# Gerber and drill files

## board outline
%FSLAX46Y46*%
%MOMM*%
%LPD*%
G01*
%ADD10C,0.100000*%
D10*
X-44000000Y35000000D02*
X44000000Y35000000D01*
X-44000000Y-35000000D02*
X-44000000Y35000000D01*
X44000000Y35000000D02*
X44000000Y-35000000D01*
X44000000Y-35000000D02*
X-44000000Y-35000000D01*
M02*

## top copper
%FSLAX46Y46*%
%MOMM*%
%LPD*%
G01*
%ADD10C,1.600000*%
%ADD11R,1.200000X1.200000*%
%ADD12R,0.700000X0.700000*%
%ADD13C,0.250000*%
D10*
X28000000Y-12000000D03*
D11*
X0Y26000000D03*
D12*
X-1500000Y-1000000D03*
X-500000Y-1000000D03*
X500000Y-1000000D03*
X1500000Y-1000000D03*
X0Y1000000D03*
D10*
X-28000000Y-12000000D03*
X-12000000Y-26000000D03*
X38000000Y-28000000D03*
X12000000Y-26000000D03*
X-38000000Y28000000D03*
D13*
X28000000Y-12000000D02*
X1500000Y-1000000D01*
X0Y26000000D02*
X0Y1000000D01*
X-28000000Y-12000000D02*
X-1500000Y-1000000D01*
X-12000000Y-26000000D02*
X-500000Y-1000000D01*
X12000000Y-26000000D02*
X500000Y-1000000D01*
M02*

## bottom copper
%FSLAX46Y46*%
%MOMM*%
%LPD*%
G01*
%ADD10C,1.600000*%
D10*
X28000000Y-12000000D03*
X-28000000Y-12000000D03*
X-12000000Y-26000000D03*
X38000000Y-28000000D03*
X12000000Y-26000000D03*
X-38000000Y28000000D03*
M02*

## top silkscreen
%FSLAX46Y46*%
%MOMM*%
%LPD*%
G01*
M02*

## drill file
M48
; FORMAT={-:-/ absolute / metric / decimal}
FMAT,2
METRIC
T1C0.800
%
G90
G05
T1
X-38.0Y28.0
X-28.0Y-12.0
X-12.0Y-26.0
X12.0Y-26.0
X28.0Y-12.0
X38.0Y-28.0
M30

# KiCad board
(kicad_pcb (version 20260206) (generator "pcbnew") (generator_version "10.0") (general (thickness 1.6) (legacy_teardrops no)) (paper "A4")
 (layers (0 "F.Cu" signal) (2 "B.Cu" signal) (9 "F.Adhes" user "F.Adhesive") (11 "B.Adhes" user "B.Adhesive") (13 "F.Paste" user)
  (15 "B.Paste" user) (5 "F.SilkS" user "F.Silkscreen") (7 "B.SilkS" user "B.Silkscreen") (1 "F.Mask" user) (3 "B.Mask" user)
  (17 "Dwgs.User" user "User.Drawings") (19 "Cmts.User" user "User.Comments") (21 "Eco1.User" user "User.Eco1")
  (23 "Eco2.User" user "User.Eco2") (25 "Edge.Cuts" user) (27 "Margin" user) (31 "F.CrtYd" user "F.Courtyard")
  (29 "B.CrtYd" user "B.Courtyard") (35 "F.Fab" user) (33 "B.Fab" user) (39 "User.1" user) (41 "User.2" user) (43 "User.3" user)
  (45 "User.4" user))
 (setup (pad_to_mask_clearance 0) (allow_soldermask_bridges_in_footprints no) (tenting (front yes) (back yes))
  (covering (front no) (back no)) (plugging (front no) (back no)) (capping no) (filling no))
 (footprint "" (layer "F.Cu") (at 28 12)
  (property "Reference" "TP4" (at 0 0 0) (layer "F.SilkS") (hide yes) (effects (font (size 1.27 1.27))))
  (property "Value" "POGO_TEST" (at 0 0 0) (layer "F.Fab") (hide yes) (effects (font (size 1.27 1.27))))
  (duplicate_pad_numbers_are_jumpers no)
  (pad "1" thru_hole circle (at 0 0) (size 1.6 1.6) (drill 0.8) (layers "*.Cu" "*.Mask") (remove_unused_layers no) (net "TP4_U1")))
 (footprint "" (layer "F.Cu") (at 0 -26)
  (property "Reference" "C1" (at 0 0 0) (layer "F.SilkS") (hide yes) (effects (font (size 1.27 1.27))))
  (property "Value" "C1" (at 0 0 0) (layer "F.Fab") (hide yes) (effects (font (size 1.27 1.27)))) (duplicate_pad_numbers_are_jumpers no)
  (pad "1" smd rect (at 0 0) (size 1.2 1.2) (layers "F.Cu" "F.Mask" "F.Paste") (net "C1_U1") (thermal_bridge_angle 45)))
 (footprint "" (layer "F.Cu") (at 0 0)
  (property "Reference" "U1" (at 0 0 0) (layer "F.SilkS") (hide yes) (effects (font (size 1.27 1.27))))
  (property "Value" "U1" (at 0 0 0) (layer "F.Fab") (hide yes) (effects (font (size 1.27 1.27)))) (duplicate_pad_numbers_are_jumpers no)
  (pad "1" smd rect (at -1.5 1) (size 0.7 0.7) (layers "F.Cu" "F.Mask" "F.Paste") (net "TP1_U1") (thermal_bridge_angle 45))
  (pad "2" smd rect (at -0.5 1) (size 0.7 0.7) (layers "F.Cu" "F.Mask" "F.Paste") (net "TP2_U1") (thermal_bridge_angle 45))
  (pad "3" smd rect (at 0.5 1) (size 0.7 0.7) (layers "F.Cu" "F.Mask" "F.Paste") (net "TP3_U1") (thermal_bridge_angle 45))
  (pad "4" smd rect (at 1.5 1) (size 0.7 0.7) (layers "F.Cu" "F.Mask" "F.Paste") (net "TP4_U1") (thermal_bridge_angle 45))
  (pad "5" smd rect (at 0 -1) (size 0.7 0.7) (layers "F.Cu" "F.Mask" "F.Paste") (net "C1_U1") (thermal_bridge_angle 45)))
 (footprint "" (layer "F.Cu") (at -28 12)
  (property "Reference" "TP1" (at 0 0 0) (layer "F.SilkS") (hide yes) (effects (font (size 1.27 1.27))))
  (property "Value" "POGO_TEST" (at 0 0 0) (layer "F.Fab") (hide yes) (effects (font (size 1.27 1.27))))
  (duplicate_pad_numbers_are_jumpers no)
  (pad "1" thru_hole circle (at 0 0) (size 1.6 1.6) (drill 0.8) (layers "*.Cu" "*.Mask") (remove_unused_layers no) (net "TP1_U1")))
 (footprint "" (layer "F.Cu") (at -12 26)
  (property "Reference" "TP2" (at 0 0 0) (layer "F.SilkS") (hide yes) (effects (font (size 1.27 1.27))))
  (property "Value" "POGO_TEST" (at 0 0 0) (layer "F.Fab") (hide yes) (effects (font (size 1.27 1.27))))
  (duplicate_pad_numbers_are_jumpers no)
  (pad "1" thru_hole circle (at 0 0) (size 1.6 1.6) (drill 0.8) (layers "*.Cu" "*.Mask") (remove_unused_layers no) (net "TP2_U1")))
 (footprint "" (layer "F.Cu") (at 38 28)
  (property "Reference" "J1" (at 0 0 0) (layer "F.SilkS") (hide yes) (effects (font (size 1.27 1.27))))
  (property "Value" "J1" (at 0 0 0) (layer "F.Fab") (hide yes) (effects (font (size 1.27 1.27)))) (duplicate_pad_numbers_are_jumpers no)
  (pad "1" thru_hole circle (at 0 0) (size 1.6 1.6) (drill 0.8) (layers "*.Cu" "*.Mask") (remove_unused_layers no) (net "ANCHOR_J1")))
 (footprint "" (layer "F.Cu") (at 12 26)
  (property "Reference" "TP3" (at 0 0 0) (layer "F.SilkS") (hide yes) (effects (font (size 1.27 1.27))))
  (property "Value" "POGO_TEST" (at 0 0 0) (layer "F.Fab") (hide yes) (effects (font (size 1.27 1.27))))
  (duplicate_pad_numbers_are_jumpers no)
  (pad "1" thru_hole circle (at 0 0) (size 1.6 1.6) (drill 0.8) (layers "*.Cu" "*.Mask") (remove_unused_layers no) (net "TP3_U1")))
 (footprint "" (layer "F.Cu") (at -38 -28)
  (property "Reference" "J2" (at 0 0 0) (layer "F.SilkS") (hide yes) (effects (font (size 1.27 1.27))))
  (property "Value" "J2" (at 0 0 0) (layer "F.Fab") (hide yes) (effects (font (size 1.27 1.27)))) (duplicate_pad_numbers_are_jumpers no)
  (pad "1" thru_hole circle (at 0 0) (size 1.6 1.6) (drill 0.8) (layers "*.Cu" "*.Mask") (remove_unused_layers no) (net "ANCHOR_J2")))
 (gr_line (start -44 -35) (end 44 -35) (stroke (width 0.1) (type default)) (layer "Edge.Cuts"))
 (gr_line (start -44 35) (end -44 -35) (stroke (width 0.1) (type default)) (layer "Edge.Cuts"))
 (gr_line (start 44 -35) (end 44 35) (stroke (width 0.1) (type default)) (layer "Edge.Cuts"))
 (gr_line (start 44 35) (end -44 35) (stroke (width 0.1) (type default)) (layer "Edge.Cuts"))
 (segment (start 28 12) (end 1.5 1) (width 0.25) (layer "F.Cu") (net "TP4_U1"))
 (segment (start 0 -26) (end 0 -1) (width 0.25) (layer "F.Cu") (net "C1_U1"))
 (segment (start -28 12) (end -1.5 1) (width 0.25) (layer "F.Cu") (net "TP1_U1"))
 (segment (start -12 26) (end -0.5 1) (width 0.25) (layer "F.Cu") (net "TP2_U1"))
 (segment (start 12 26) (end 0.5 1) (width 0.25) (layer "F.Cu") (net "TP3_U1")))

